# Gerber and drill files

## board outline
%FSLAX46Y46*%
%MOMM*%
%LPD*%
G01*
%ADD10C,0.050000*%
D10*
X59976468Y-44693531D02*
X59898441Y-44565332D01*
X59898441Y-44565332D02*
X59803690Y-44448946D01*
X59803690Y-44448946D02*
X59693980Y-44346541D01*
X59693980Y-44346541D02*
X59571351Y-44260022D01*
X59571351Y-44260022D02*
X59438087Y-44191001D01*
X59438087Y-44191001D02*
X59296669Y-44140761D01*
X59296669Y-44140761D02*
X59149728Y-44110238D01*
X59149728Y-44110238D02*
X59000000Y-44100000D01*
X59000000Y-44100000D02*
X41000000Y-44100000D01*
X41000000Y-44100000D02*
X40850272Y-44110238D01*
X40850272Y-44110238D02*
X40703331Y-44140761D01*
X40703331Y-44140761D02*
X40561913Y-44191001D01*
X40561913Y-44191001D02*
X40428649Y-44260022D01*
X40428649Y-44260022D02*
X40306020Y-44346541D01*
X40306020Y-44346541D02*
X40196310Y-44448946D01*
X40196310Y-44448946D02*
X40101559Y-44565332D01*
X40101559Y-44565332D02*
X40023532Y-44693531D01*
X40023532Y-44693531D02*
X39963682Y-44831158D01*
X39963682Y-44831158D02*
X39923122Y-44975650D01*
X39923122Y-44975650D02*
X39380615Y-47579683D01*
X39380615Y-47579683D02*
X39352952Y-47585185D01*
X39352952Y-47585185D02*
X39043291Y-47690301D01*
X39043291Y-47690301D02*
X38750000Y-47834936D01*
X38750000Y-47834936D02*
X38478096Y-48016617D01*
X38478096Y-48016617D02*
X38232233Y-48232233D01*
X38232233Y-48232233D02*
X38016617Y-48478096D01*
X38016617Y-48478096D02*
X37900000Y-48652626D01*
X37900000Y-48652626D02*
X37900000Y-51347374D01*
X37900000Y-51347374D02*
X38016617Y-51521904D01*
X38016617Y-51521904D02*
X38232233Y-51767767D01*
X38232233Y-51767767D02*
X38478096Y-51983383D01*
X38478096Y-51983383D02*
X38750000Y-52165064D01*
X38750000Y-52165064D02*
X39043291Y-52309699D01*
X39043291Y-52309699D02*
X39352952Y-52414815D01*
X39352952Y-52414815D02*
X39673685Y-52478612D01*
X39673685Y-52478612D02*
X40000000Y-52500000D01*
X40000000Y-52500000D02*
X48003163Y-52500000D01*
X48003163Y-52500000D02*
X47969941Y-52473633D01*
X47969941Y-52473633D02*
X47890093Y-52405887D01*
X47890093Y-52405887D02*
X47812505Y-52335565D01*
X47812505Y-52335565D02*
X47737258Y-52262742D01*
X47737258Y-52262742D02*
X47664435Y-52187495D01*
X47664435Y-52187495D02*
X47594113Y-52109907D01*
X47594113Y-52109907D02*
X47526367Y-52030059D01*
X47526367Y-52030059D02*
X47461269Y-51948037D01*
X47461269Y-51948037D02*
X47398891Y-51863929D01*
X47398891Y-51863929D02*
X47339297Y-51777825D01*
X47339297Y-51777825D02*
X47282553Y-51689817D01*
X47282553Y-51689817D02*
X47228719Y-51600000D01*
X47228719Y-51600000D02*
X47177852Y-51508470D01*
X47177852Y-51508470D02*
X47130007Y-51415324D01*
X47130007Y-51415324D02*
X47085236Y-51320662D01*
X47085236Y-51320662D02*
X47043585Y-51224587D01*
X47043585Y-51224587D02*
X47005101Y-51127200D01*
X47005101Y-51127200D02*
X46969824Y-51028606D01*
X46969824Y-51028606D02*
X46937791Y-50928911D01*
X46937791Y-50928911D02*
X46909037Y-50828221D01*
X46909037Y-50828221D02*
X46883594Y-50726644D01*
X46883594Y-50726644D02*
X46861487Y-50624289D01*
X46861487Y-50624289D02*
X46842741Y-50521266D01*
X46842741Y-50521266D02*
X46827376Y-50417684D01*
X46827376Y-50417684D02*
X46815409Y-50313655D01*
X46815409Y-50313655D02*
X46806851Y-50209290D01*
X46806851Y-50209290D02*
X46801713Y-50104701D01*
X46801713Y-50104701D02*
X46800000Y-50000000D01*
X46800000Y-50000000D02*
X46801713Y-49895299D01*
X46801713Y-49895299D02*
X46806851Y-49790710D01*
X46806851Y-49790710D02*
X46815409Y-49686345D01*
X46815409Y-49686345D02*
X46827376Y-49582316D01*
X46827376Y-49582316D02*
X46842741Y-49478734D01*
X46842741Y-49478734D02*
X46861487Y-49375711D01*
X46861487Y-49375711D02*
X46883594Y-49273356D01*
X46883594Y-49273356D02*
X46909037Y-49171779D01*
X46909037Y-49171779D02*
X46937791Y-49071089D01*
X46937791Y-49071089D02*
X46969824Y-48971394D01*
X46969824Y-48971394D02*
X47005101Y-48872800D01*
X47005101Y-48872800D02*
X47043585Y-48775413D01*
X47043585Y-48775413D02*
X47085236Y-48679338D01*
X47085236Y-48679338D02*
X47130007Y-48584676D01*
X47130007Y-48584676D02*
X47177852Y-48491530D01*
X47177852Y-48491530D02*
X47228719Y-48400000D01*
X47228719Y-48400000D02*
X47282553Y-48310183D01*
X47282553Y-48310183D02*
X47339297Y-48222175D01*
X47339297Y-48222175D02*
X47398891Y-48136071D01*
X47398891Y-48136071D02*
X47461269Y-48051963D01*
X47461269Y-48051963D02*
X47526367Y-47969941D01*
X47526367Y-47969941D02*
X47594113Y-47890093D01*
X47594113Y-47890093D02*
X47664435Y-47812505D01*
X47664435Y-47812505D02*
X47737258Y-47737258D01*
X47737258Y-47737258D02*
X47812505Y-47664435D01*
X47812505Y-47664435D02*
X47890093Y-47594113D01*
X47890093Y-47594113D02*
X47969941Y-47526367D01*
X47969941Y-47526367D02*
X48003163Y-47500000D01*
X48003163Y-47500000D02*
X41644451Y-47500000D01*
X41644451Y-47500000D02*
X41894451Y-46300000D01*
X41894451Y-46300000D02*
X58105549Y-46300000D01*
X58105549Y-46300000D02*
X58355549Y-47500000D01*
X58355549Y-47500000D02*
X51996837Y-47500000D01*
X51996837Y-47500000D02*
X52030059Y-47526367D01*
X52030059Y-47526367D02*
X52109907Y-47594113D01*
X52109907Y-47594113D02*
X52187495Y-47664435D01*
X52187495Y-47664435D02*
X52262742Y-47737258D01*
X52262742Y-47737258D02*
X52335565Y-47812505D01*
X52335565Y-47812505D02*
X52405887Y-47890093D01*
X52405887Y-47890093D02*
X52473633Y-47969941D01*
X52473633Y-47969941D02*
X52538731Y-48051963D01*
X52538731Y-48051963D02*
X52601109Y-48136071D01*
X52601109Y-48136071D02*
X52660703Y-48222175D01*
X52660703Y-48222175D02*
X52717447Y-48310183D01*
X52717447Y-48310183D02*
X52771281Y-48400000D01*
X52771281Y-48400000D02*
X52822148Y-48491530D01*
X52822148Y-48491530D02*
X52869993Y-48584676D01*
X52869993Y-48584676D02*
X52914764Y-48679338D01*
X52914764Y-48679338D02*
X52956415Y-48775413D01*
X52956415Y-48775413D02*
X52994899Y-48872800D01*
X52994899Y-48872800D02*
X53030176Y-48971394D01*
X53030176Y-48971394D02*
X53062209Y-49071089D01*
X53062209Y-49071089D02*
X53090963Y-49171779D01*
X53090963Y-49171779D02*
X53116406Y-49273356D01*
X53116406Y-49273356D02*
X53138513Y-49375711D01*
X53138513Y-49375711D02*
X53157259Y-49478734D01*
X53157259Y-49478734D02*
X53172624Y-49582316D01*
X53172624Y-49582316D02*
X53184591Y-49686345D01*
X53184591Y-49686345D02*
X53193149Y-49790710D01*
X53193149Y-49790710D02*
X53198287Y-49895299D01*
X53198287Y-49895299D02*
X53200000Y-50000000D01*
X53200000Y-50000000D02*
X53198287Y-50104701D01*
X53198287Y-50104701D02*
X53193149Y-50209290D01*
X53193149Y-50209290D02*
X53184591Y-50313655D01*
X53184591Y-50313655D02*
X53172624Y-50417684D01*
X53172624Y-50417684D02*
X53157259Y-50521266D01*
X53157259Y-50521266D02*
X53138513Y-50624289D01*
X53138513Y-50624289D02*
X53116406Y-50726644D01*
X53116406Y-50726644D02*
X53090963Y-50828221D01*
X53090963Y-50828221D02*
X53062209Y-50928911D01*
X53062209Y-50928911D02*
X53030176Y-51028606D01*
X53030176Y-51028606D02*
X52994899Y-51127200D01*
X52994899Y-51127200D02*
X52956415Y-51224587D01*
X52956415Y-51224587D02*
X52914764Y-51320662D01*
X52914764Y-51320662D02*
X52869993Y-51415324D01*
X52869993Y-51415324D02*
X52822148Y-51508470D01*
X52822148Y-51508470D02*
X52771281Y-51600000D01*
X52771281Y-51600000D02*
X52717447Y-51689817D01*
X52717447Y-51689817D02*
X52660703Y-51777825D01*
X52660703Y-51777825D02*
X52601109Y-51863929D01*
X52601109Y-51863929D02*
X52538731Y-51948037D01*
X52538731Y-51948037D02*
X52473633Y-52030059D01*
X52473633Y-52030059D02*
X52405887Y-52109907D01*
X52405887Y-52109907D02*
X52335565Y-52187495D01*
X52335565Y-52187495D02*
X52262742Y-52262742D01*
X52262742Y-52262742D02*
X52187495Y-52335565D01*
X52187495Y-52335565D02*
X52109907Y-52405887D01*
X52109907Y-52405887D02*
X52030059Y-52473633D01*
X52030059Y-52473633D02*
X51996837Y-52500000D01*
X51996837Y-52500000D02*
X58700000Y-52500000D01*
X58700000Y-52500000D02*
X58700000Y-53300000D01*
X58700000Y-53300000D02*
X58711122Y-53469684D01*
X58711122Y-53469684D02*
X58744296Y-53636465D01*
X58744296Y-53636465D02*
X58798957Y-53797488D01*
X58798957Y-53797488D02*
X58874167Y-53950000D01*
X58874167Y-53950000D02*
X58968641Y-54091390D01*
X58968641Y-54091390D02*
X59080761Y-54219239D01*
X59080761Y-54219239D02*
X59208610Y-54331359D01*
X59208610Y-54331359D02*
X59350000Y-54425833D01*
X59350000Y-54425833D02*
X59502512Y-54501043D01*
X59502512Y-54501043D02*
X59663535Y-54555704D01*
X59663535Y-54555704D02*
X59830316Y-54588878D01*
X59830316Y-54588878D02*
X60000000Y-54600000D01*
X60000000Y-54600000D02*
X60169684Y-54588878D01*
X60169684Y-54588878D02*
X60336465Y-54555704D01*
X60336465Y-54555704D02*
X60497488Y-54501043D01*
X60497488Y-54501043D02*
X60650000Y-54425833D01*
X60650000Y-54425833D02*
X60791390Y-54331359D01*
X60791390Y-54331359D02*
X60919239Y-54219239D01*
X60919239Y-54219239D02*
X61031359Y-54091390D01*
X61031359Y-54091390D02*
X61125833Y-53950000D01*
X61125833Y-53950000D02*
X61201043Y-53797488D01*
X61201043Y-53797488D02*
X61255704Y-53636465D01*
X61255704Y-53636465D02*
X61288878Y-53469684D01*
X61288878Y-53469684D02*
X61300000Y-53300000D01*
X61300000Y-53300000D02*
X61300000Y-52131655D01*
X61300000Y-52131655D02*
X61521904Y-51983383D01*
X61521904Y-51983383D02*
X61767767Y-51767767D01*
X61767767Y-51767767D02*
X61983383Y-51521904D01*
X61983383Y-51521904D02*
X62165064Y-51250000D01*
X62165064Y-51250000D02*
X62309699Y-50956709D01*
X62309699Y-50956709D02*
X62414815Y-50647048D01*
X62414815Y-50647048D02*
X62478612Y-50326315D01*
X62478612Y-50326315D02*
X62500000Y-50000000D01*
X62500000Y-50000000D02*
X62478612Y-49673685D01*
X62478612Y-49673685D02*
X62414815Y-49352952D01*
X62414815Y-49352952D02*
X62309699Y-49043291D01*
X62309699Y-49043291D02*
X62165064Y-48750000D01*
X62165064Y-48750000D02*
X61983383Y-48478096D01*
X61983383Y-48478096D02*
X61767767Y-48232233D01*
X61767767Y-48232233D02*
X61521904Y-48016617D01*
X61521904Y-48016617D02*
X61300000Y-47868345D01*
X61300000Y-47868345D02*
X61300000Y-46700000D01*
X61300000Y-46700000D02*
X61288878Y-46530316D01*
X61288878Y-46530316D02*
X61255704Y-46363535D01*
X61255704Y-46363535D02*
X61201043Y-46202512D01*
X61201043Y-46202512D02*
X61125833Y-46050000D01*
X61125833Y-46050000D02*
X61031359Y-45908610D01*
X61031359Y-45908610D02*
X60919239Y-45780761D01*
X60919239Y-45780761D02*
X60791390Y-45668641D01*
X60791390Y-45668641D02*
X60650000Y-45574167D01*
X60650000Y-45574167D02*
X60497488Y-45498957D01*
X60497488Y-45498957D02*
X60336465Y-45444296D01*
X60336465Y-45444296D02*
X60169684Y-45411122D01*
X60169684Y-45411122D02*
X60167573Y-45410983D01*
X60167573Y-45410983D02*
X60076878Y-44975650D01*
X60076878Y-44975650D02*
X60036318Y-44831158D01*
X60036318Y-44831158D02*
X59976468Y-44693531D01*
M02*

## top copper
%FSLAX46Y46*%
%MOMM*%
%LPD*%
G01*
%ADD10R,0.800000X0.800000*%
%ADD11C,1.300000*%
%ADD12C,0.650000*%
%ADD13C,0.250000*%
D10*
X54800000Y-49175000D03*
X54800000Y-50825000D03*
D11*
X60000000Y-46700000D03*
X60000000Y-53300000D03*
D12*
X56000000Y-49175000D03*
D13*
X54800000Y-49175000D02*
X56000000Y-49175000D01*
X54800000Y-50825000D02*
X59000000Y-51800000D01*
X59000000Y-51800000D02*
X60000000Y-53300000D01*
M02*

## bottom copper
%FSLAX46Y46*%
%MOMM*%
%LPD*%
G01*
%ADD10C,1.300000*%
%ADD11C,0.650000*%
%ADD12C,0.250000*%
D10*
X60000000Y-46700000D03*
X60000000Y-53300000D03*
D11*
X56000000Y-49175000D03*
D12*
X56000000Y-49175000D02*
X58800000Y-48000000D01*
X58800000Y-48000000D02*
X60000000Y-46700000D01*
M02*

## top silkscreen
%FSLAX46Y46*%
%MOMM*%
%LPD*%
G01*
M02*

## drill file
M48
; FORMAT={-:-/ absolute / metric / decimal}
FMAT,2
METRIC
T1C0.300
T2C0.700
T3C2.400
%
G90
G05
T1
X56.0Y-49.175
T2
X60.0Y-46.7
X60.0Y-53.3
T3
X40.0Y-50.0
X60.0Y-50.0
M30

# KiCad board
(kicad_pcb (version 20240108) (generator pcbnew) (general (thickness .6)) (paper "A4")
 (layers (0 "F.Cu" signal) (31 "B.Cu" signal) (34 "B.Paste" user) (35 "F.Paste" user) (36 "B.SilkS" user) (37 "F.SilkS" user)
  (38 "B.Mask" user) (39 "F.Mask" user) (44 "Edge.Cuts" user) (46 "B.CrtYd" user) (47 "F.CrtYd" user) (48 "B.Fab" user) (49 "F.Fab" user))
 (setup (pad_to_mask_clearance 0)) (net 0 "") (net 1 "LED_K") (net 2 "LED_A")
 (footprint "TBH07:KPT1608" (layer "F.Cu") (at 54.8 50)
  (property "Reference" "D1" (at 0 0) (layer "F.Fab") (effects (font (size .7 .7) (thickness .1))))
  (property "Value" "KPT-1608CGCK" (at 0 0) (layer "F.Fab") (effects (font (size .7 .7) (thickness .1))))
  (pad "1" smd rect (at 0 -.825) (size .8 .8) (layers "F.Cu" "F.Paste" "F.Mask") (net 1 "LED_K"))
  (pad "2" smd rect (at 0 .825) (size .8 .8) (layers "F.Cu" "F.Paste" "F.Mask") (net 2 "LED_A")))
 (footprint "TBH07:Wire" (layer "F.Cu") (at 60 46.7)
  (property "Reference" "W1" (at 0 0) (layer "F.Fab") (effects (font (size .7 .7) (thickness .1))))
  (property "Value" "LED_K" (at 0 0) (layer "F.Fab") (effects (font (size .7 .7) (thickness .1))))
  (pad "1" thru_hole circle (at 0 0) (size 1.3 1.3) (drill .7) (layers "*.Cu" "*.Mask") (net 1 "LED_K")))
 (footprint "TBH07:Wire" (layer "F.Cu") (at 60 53.3)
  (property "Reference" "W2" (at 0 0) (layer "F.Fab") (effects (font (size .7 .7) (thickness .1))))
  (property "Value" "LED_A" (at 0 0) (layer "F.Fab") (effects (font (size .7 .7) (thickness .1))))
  (pad "1" thru_hole circle (at 0 0) (size 1.3 1.3) (drill .7) (layers "*.Cu" "*.Mask") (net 2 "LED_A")))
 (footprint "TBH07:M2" (layer "F.Cu") (at 40 50)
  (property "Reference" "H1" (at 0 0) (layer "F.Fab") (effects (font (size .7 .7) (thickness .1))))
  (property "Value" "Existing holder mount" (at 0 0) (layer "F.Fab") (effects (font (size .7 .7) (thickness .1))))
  (pad "" np_thru_hole circle (at 0 0) (size 2.4 2.4) (drill 2.4) (layers "*.Cu" "*.Mask")))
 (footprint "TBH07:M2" (layer "F.Cu") (at 60 50)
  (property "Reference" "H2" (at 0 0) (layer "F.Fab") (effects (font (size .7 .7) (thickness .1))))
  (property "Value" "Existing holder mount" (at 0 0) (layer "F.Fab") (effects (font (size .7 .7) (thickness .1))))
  (pad "" np_thru_hole circle (at 0 0) (size 2.4 2.4) (drill 2.4) (layers "*.Cu" "*.Mask")))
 (segment (start 54.8 49.175) (end 56 49.175) (width .25) (layer "F.Cu") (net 1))
 (via (at 56 49.175) (size .65) (drill .3) (layers "F.Cu" "B.Cu") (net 1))
 (segment (start 56 49.175) (end 58.8 48.0) (width .25) (layer "B.Cu") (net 1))
 (segment (start 58.8 48.0) (end 60 46.7) (width .25) (layer "B.Cu") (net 1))
 (segment (start 54.8 50.825) (end 59.0 51.8) (width .25) (layer "F.Cu") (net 2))
 (segment (start 59.0 51.8) (end 60 53.3) (width .25) (layer "F.Cu") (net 2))
 (gr_line (start 59.97646762268844 44.69353086782984) (end 59.89844084614742 44.56533154641664) (stroke (width .05) (type default))
  (layer "Edge.Cuts"))
 (gr_line (start 59.89844084614742 44.56533154641664) (end 59.80369026607012 44.448946102983186) (stroke (width .05) (type default))
  (layer "Edge.Cuts"))
 (gr_line (start 59.80369026607012 44.448946102983186) (end 59.69397959354886 44.34654096540152) (stroke (width .05) (type default))
  (layer "Edge.Cuts"))
 (gr_line (start 59.69397959354886 44.34654096540152) (end 59.57135101059367 44.26002232861967) (stroke (width .05) (type default))
  (layer "Edge.Cuts"))
 (gr_line (start 59.57135101059367 44.26002232861967) (end 59.4380871564435 44.19100067227017) (stroke (width .05) (type default))
  (layer "Edge.Cuts"))
 (gr_line (start 59.4380871564435 44.19100067227017) (end 59.29666863794614 44.14076078279778) (stroke (width .05) (type default))
  (layer "Edge.Cuts"))
 (gr_line (start 59.29666863794614 44.14076078279778) (end 59.14972785491944 44.110237838121904) (stroke (width .05) (type default))
  (layer "Edge.Cuts"))
 (gr_line (start 59.14972785491944 44.110237838121904) (end 59.0 44.1) (stroke (width .05) (type default)) (layer "Edge.Cuts"))
 (gr_line (start 59.0 44.1) (end 41.0 44.1) (stroke (width .05) (type default)) (layer "Edge.Cuts"))
 (gr_line (start 41.0 44.1) (end 40.85027214508056 44.110237838121904) (stroke (width .05) (type default)) (layer "Edge.Cuts"))
 (gr_line (start 40.85027214508056 44.110237838121904) (end 40.70333136205386 44.14076078279778) (stroke (width .05) (type default))
  (layer "Edge.Cuts"))
 (gr_line (start 40.70333136205386 44.14076078279778) (end 40.5619128435565 44.19100067227017) (stroke (width .05) (type default))
  (layer "Edge.Cuts"))
 (gr_line (start 40.5619128435565 44.19100067227017) (end 40.42864898940633 44.26002232861967) (stroke (width .05) (type default))
  (layer "Edge.Cuts"))
 (gr_line (start 40.42864898940633 44.26002232861967) (end 40.30602040645114 44.34654096540152) (stroke (width .05) (type default))
  (layer "Edge.Cuts"))
 (gr_line (start 40.30602040645114 44.34654096540152) (end 40.19630973392988 44.448946102983186) (stroke (width .05) (type default))
  (layer "Edge.Cuts"))
 (gr_line (start 40.19630973392988 44.448946102983186) (end 40.10155915385258 44.56533154641664) (stroke (width .05) (type default))
  (layer "Edge.Cuts"))
 (gr_line (start 40.10155915385258 44.56533154641664) (end 40.02353237731156 44.69353086782984) (stroke (width .05) (type default))
  (layer "Edge.Cuts"))
 (gr_line (start 40.02353237731156 44.69353086782984) (end 39.9636818143203 44.831157732859225) (stroke (width .05) (type default))
  (layer "Edge.Cuts"))
 (gr_line (start 39.9636818143203 44.831157732859225) (end 39.92312153828863 44.9756503204768) (stroke (width .05) (type default))
  (layer "Edge.Cuts"))
 (gr_line (start 39.92312153828863 44.9756503204768) (end 39.3806147187135 47.57968305443743) (stroke (width .05) (type default))
  (layer "Edge.Cuts"))
 (gr_line (start 39.3806147187135 47.57968305443743) (end 39.3529523872437 47.58518543427733) (stroke (width .05) (type default))
  (layer "Edge.Cuts"))
 (gr_line (start 39.3529523872437 47.58518543427733) (end 39.043291419087275 47.69030116872178) (stroke (width .05) (type default))
  (layer "Edge.Cuts"))
 (gr_line (start 39.043291419087275 47.69030116872178) (end 38.75 47.8349364905389) (stroke (width .05) (type default)) (layer "Edge.Cuts"))
 (gr_line (start 38.75 47.8349364905389) (end 38.4780964274782 48.01661664927191) (stroke (width .05) (type default)) (layer "Edge.Cuts"))
 (gr_line (start 38.4780964274782 48.01661664927191) (end 38.23223304703363 48.23223304703363) (stroke (width .05) (type default))
  (layer "Edge.Cuts"))
 (gr_line (start 38.23223304703363 48.23223304703363) (end 38.01661664927191 48.4780964274782) (stroke (width .05) (type default))
  (layer "Edge.Cuts"))
 (gr_line (start 38.01661664927191 48.4780964274782) (end 37.9 48.652625576801285) (stroke (width .05) (type default)) (layer "Edge.Cuts"))
 (gr_line (start 37.9 48.652625576801285) (end 37.9 51.347374423198715) (stroke (width .05) (type default)) (layer "Edge.Cuts"))
 (gr_line (start 37.9 51.347374423198715) (end 38.01661664927191 51.5219035725218) (stroke (width .05) (type default)) (layer "Edge.Cuts"))
 (gr_line (start 38.01661664927191 51.5219035725218) (end 38.23223304703363 51.76776695296637) (stroke (width .05) (type default))
  (layer "Edge.Cuts"))
 (gr_line (start 38.23223304703363 51.76776695296637) (end 38.4780964274782 51.98338335072809) (stroke (width .05) (type default))
  (layer "Edge.Cuts"))
 (gr_line (start 38.4780964274782 51.98338335072809) (end 38.75 52.1650635094611) (stroke (width .05) (type default)) (layer "Edge.Cuts"))
 (gr_line (start 38.75 52.1650635094611) (end 39.043291419087275 52.30969883127822) (stroke (width .05) (type default)) (layer "Edge.Cuts"))
 (gr_line (start 39.043291419087275 52.30969883127822) (end 39.3529523872437 52.41481456572267) (stroke (width .05) (type default))
  (layer "Edge.Cuts"))
 (gr_line (start 39.3529523872437 52.41481456572267) (end 39.67368451944987 52.478612153434526) (stroke (width .05) (type default))
  (layer "Edge.Cuts"))
 (gr_line (start 39.67368451944987 52.478612153434526) (end 40.0 52.5) (stroke (width .05) (type default)) (layer "Edge.Cuts"))
 (gr_line (start 40.0 52.5) (end 48.00316310634037 52.5) (stroke (width .05) (type default)) (layer "Edge.Cuts"))
 (gr_line (start 48.00316310634037 52.5) (end 47.969941490676334 52.47363345076076) (stroke (width .05) (type default)) (layer "Edge.Cuts"))
 (gr_line (start 47.969941490676334 52.47363345076076) (end 47.89009339167978 52.40588738393273) (stroke (width .05) (type default))
  (layer "Edge.Cuts"))
 (gr_line (start 47.89009339167978 52.40588738393273) (end 47.812504633526814 52.33556503263307) (stroke (width .05) (type default))
  (layer "Edge.Cuts"))
 (gr_line (start 47.812504633526814 52.33556503263307) (end 47.737258300203045 52.26274169979695) (stroke (width .05) (type default))
  (layer "Edge.Cuts"))
 (gr_line (start 47.737258300203045 52.26274169979695) (end 47.66443496736692 52.187495366473186) (stroke (width .05) (type default))
  (layer "Edge.Cuts"))
 (gr_line (start 47.66443496736692 52.187495366473186) (end 47.59411261606727 52.109906608320216) (stroke (width .05) (type default))
  (layer "Edge.Cuts"))
 (gr_line (start 47.59411261606727 52.109906608320216) (end 47.52636654923924 52.030058509323666) (stroke (width .05) (type default))
  (layer "Edge.Cuts"))
 (gr_line (start 47.52636654923924 52.030058509323666) (end 47.461269311068044 51.9480365728279) (stroke (width .05) (type default))
  (layer "Edge.Cuts"))
 (gr_line (start 47.461269311068044 51.9480365728279) (end 47.39889060930683 51.86392862997697) (stroke (width .05) (type default))
  (layer "Edge.Cuts"))
 (gr_line (start 47.39889060930683 51.86392862997697) (end 47.33929724063185 51.77782474566273) (stroke (width .05) (type default))
  (layer "Edge.Cuts"))
 (gr_line (start 47.33929724063185 51.77782474566273) (end 47.28255301911494 51.68981712208117) (stroke (width .05) (type default))
  (layer "Edge.Cuts"))
 (gr_line (start 47.28255301911494 51.68981712208117) (end 47.2287187078898 51.6) (stroke (width .05) (type default)) (layer "Edge.Cuts"))
 (gr_line (start 47.2287187078898 51.6) (end 47.17785195408526 51.50846955784319) (stroke (width .05) (type default)) (layer "Edge.Cuts"))
 (gr_line (start 47.17785195408526 51.50846955784319) (end 47.1300072270954 51.415323808700805) (stroke (width .05) (type default))
  (layer "Edge.Cuts"))
 (gr_line (start 47.1300072270954 51.415323808700805) (end 47.08523576025224 51.320662495374066) (stroke (width .05) (type default))
  (layer "Edge.Cuts"))
 (gr_line (start 47.08523576025224 51.320662495374066) (end 47.04358549596388 51.22458698356829) (stroke (width .05) (type default))
  (layer "Edge.Cuts"))
 (gr_line (start 47.04358549596388 51.22458698356829) (end 47.00510103437656 51.12720015334795) (stroke (width .05) (type default))
  (layer "Edge.Cuts"))
 (gr_line (start 47.00510103437656 51.12720015334795) (end 46.969823585615664 51.02860628897012) (stroke (width .05) (type default))
  (layer "Edge.Cuts"))
 (gr_line (start 46.969823585615664 51.02860628897012) (end 46.937790925656934 50.92891096721428) (stroke (width .05) (type default))
  (layer "Edge.Cuts"))
 (gr_line (start 46.937790925656934 50.92891096721428) (end 46.90903735587498 50.828220944328066) (stroke (width .05) (type default))
  (layer "Edge.Cuts"))
 (gr_line (start 46.90903735587498 50.828220944328066) (end 46.883593666312535 50.726644041709996) (stroke (width .05) (type default))
  (layer "Edge.Cuts"))
 (gr_line (start 46.883593666312535 50.726644041709996) (end 46.86148710270966 50.62428903045161) (stroke (width .05) (type default))
  (layer "Edge.Cuts"))
 (gr_line (start 46.86148710270966 50.62428903045161) (end 46.842741337328384 50.521265514862684) (stroke (width .05) (type default))
  (layer "Edge.Cuts"))
 (gr_line (start 46.842741337328384 50.521265514862684) (end 46.827376443603804 50.41768381510416) (stroke (width .05) (type default))
  (layer "Edge.Cuts"))
 (gr_line (start 46.827376443603804 50.41768381510416) (end 46.815408874648966 50.31365484905459) (stroke (width .05) (type default))
  (layer "Edge.Cuts"))
 (gr_line (start 46.815408874648966 50.31365484905459) (end 46.80685144563647 50.20929001353646) (stroke (width .05) (type default))
  (layer "Edge.Cuts"))
 (gr_line (start 46.80685144563647 50.20929001353646) (end 46.80171332007563 50.10470106502968) (stroke (width .05) (type default))
  (layer "Edge.Cuts"))
 (gr_line (start 46.80171332007563 50.10470106502968) (end 46.8 50.0) (stroke (width .05) (type default)) (layer "Edge.Cuts"))
 (gr_line (start 46.8 50.0) (end 46.80171332007563 49.89529893497031) (stroke (width .05) (type default)) (layer "Edge.Cuts"))
 (gr_line (start 46.80171332007563 49.89529893497031) (end 46.80685144563647 49.79070998646354) (stroke (width .05) (type default))
  (layer "Edge.Cuts"))
 (gr_line (start 46.80685144563647 49.79070998646354) (end 46.815408874648966 49.68634515094541) (stroke (width .05) (type default))
  (layer "Edge.Cuts"))
 (gr_line (start 46.815408874648966 49.68634515094541) (end 46.827376443603804 49.58231618489583) (stroke (width .05) (type default))
  (layer "Edge.Cuts"))
 (gr_line (start 46.827376443603804 49.58231618489583) (end 46.842741337328384 49.478734485137316) (stroke (width .05) (type default))
  (layer "Edge.Cuts"))
 (gr_line (start 46.842741337328384 49.478734485137316) (end 46.86148710270966 49.375710969548386) (stroke (width .05) (type default))
  (layer "Edge.Cuts"))
 (gr_line (start 46.86148710270966 49.375710969548386) (end 46.883593666312535 49.273355958290004) (stroke (width .05) (type default))
  (layer "Edge.Cuts"))
 (gr_line (start 46.883593666312535 49.273355958290004) (end 46.90903735587498 49.171779055671934) (stroke (width .05) (type default))
  (layer "Edge.Cuts"))
 (gr_line (start 46.90903735587498 49.171779055671934) (end 46.937790925656934 49.07108903278572) (stroke (width .05) (type default))
  (layer "Edge.Cuts"))
 (gr_line (start 46.937790925656934 49.07108903278572) (end 46.969823585615664 48.97139371102988) (stroke (width .05) (type default))
  (layer "Edge.Cuts"))
 (gr_line (start 46.969823585615664 48.97139371102988) (end 47.00510103437656 48.87279984665205) (stroke (width .05) (type default))
  (layer "Edge.Cuts"))
 (gr_line (start 47.00510103437656 48.87279984665205) (end 47.04358549596388 48.77541301643171) (stroke (width .05) (type default))
  (layer "Edge.Cuts"))
 (gr_line (start 47.04358549596388 48.77541301643171) (end 47.08523576025224 48.679337504625934) (stroke (width .05) (type default))
  (layer "Edge.Cuts"))
 (gr_line (start 47.08523576025224 48.679337504625934) (end 47.1300072270954 48.584676191299195) (stroke (width .05) (type default))
  (layer "Edge.Cuts"))
 (gr_line (start 47.1300072270954 48.584676191299195) (end 47.17785195408526 48.49153044215681) (stroke (width .05) (type default))
  (layer "Edge.Cuts"))
 (gr_line (start 47.17785195408526 48.49153044215681) (end 47.2287187078898 48.4) (stroke (width .05) (type default)) (layer "Edge.Cuts"))
 (gr_line (start 47.2287187078898 48.4) (end 47.28255301911495 48.31018287791882) (stroke (width .05) (type default)) (layer "Edge.Cuts"))
 (gr_line (start 47.28255301911495 48.31018287791882) (end 47.33929724063186 48.22217525433727) (stroke (width .05) (type default))
  (layer "Edge.Cuts"))
 (gr_line (start 47.33929724063186 48.22217525433727) (end 47.39889060930683 48.13607137002303) (stroke (width .05) (type default))
  (layer "Edge.Cuts"))
 (gr_line (start 47.39889060930683 48.13607137002303) (end 47.46126931106805 48.05196342717209) (stroke (width .05) (type default))
  (layer "Edge.Cuts"))
 (gr_line (start 47.46126931106805 48.05196342717209) (end 47.52636654923924 47.969941490676334) (stroke (width .05) (type default))
  (layer "Edge.Cuts"))
 (gr_line (start 47.52636654923924 47.969941490676334) (end 47.59411261606727 47.89009339167978) (stroke (width .05) (type default))
  (layer "Edge.Cuts"))
 (gr_line (start 47.59411261606727 47.89009339167978) (end 47.66443496736693 47.812504633526814) (stroke (width .05) (type default))
  (layer "Edge.Cuts"))
 (gr_line (start 47.66443496736693 47.812504633526814) (end 47.737258300203045 47.737258300203045) (stroke (width .05) (type default))
  (layer "Edge.Cuts"))
 (gr_line (start 47.737258300203045 47.737258300203045) (end 47.812504633526814 47.66443496736692) (stroke (width .05) (type default))
  (layer "Edge.Cuts"))
 (gr_line (start 47.812504633526814 47.66443496736692) (end 47.890093391679784 47.59411261606727) (stroke (width .05) (type default))
  (layer "Edge.Cuts"))
 (gr_line (start 47.890093391679784 47.59411261606727) (end 47.969941490676334 47.52636654923924) (stroke (width .05) (type default))
  (layer "Edge.Cuts"))
 (gr_line (start 47.969941490676334 47.52636654923924) (end 48.00316310634037 47.5) (stroke (width .05) (type default)) (layer "Edge.Cuts"))
 (gr_line (start 48.00316310634037 47.5) (end 41.64445131161203 47.5) (stroke (width .05) (type default)) (layer "Edge.Cuts"))
 (gr_line (start 41.64445131161203 47.5) (end 41.89445131161203 46.3) (stroke (width .05) (type default)) (layer "Edge.Cuts"))
 (gr_line (start 41.89445131161203 46.3) (end 58.10554868838797 46.3) (stroke (width .05) (type default)) (layer "Edge.Cuts"))
 (gr_line (start 58.10554868838797 46.3) (end 58.35554868838797 47.5) (stroke (width .05) (type default)) (layer "Edge.Cuts"))
 (gr_line (start 58.35554868838797 47.5) (end 51.99683689365963 47.5) (stroke (width .05) (type default)) (layer "Edge.Cuts"))
 (gr_line (start 51.99683689365963 47.5) (end 52.030058509323666 47.52636654923924) (stroke (width .05) (type default)) (layer "Edge.Cuts"))
 (gr_line (start 52.030058509323666 47.52636654923924) (end 52.10990660832022 47.59411261606727) (stroke (width .05) (type default))
  (layer "Edge.Cuts"))
 (gr_line (start 52.10990660832022 47.59411261606727) (end 52.187495366473186 47.66443496736693) (stroke (width .05) (type default))
  (layer "Edge.Cuts"))
 (gr_line (start 52.187495366473186 47.66443496736693) (end 52.262741699796955 47.737258300203045) (stroke (width .05) (type default))
  (layer "Edge.Cuts"))
 (gr_line (start 52.262741699796955 47.737258300203045) (end 52.33556503263308 47.812504633526814) (stroke (width .05) (type default))
  (layer "Edge.Cuts"))
 (gr_line (start 52.33556503263308 47.812504633526814) (end 52.40588738393273 47.89009339167978) (stroke (width .05) (type default))
  (layer "Edge.Cuts"))
 (gr_line (start 52.40588738393273 47.89009339167978) (end 52.47363345076076 47.969941490676334) (stroke (width .05) (type default))
  (layer "Edge.Cuts"))
 (gr_line (start 52.47363345076076 47.969941490676334) (end 52.538730688931956 48.0519634271721) (stroke (width .05) (type default))
  (layer "Edge.Cuts"))
 (gr_line (start 52.538730688931956 48.0519634271721) (end 52.60110939069317 48.13607137002303) (stroke (width .05) (type default))
  (layer "Edge.Cuts"))
 (gr_line (start 52.60110939069317 48.13607137002303) (end 52.66070275936814 48.22217525433727) (stroke (width .05) (type default))
  (layer "Edge.Cuts"))
 (gr_line (start 52.66070275936814 48.22217525433727) (end 52.71744698088505 48.31018287791882) (stroke (width .05) (type default))
  (layer "Edge.Cuts"))
 (gr_line (start 52.71744698088505 48.31018287791882) (end 52.7712812921102 48.4) (stroke (width .05) (type default)) (layer "Edge.Cuts"))
 (gr_line (start 52.7712812921102 48.4) (end 52.82214804591474 48.49153044215681) (stroke (width .05) (type default)) (layer "Edge.Cuts"))
 (gr_line (start 52.82214804591474 48.49153044215681) (end 52.8699927729046 48.584676191299195) (stroke (width .05) (type default))
  (layer "Edge.Cuts"))
 (gr_line (start 52.8699927729046 48.584676191299195) (end 52.91476423974776 48.679337504625934) (stroke (width .05) (type default))
  (layer "Edge.Cuts"))
 (gr_line (start 52.91476423974776 48.679337504625934) (end 52.95641450403612 48.77541301643171) (stroke (width .05) (type default))
  (layer "Edge.Cuts"))
 (gr_line (start 52.95641450403612 48.77541301643171) (end 52.99489896562344 48.87279984665205) (stroke (width .05) (type default))
  (layer "Edge.Cuts"))
 (gr_line (start 52.99489896562344 48.87279984665205) (end 53.030176414384336 48.97139371102988) (stroke (width .05) (type default))
  (layer "Edge.Cuts"))
 (gr_line (start 53.030176414384336 48.97139371102988) (end 53.062209074343066 49.07108903278572) (stroke (width .05) (type default))
  (layer "Edge.Cuts"))
 (gr_line (start 53.062209074343066 49.07108903278572) (end 53.09096264412502 49.171779055671934) (stroke (width .05) (type default))
  (layer "Edge.Cuts"))
 (gr_line (start 53.09096264412502 49.171779055671934) (end 53.116406333687465 49.273355958290004) (stroke (width .05) (type default))
  (layer "Edge.Cuts"))
 (gr_line (start 53.116406333687465 49.273355958290004) (end 53.13851289729034 49.375710969548386) (stroke (width .05) (type default))
  (layer "Edge.Cuts"))
 (gr_line (start 53.13851289729034 49.375710969548386) (end 53.157258662671616 49.478734485137316) (stroke (width .05) (type default))
  (layer "Edge.Cuts"))
 (gr_line (start 53.157258662671616 49.478734485137316) (end 53.172623556396196 49.58231618489584) (stroke (width .05) (type default))
  (layer "Edge.Cuts"))
 (gr_line (start 53.172623556396196 49.58231618489584) (end 53.184591125351034 49.68634515094541) (stroke (width .05) (type default))
  (layer "Edge.Cuts"))
 (gr_line (start 53.184591125351034 49.68634515094541) (end 53.19314855436353 49.79070998646354) (stroke (width .05) (type default))
  (layer "Edge.Cuts"))
 (gr_line (start 53.19314855436353 49.79070998646354) (end 53.19828667992437 49.89529893497031) (stroke (width .05) (type default))
  (layer "Edge.Cuts"))
 (gr_line (start 53.19828667992437 49.89529893497031) (end 53.2 50.0) (stroke (width .05) (type default)) (layer "Edge.Cuts"))
 (gr_line (start 53.2 50.0) (end 53.19828667992437 50.10470106502969) (stroke (width .05) (type default)) (layer "Edge.Cuts"))
 (gr_line (start 53.19828667992437 50.10470106502969) (end 53.19314855436353 50.20929001353646) (stroke (width .05) (type default))
  (layer "Edge.Cuts"))
 (gr_line (start 53.19314855436353 50.20929001353646) (end 53.184591125351034 50.31365484905459) (stroke (width .05) (type default))
  (layer "Edge.Cuts"))
 (gr_line (start 53.184591125351034 50.31365484905459) (end 53.17262355639619 50.41768381510417) (stroke (width .05) (type default))
  (layer "Edge.Cuts"))
 (gr_line (start 53.17262355639619 50.41768381510417) (end 53.157258662671616 50.521265514862684) (stroke (width .05) (type default))
  (layer "Edge.Cuts"))
 (gr_line (start 53.157258662671616 50.521265514862684) (end 53.13851289729034 50.624289030451614) (stroke (width .05) (type default))
  (layer "Edge.Cuts"))
 (gr_line (start 53.13851289729034 50.624289030451614) (end 53.116406333687465 50.726644041709996) (stroke (width .05) (type default))
  (layer "Edge.Cuts"))
 (gr_line (start 53.116406333687465 50.726644041709996) (end 53.09096264412502 50.828220944328066) (stroke (width .05) (type default))
  (layer "Edge.Cuts"))
 (gr_line (start 53.09096264412502 50.828220944328066) (end 53.062209074343066 50.928910967214286) (stroke (width .05) (type default))
  (layer "Edge.Cuts"))
 (gr_line (start 53.062209074343066 50.928910967214286) (end 53.030176414384336 51.02860628897012) (stroke (width .05) (type default))
  (layer "Edge.Cuts"))
 (gr_line (start 53.030176414384336 51.02860628897012) (end 52.99489896562344 51.12720015334795) (stroke (width .05) (type default))
  (layer "Edge.Cuts"))
 (gr_line (start 52.99489896562344 51.12720015334795) (end 52.95641450403612 51.22458698356829) (stroke (width .05) (type default))
  (layer "Edge.Cuts"))
 (gr_line (start 52.95641450403612 51.22458698356829) (end 52.91476423974776 51.320662495374066) (stroke (width .05) (type default))
  (layer "Edge.Cuts"))
 (gr_line (start 52.91476423974776 51.320662495374066) (end 52.8699927729046 51.415323808700805) (stroke (width .05) (type default))
  (layer "Edge.Cuts"))
 (gr_line (start 52.8699927729046 51.415323808700805) (end 52.82214804591474 51.50846955784319) (stroke (width .05) (type default))
  (layer "Edge.Cuts"))
 (gr_line (start 52.82214804591474 51.50846955784319) (end 52.7712812921102 51.6) (stroke (width .05) (type default)) (layer "Edge.Cuts"))
 (gr_line (start 52.7712812921102 51.6) (end 52.71744698088505 51.68981712208118) (stroke (width .05) (type default)) (layer "Edge.Cuts"))
 (gr_line (start 52.71744698088505 51.68981712208118) (end 52.66070275936814 51.77782474566273) (stroke (width .05) (type default))
  (layer "Edge.Cuts"))
 (gr_line (start 52.66070275936814 51.77782474566273) (end 52.60110939069317 51.86392862997697) (stroke (width .05) (type default))
  (layer "Edge.Cuts"))
 (gr_line (start 52.60110939069317 51.86392862997697) (end 52.53873068893195 51.94803657282791) (stroke (width .05) (type default))
  (layer "Edge.Cuts"))
 (gr_line (start 52.53873068893195 51.94803657282791) (end 52.47363345076076 52.030058509323666) (stroke (width .05) (type default))
  (layer "Edge.Cuts"))
 (gr_line (start 52.47363345076076 52.030058509323666) (end 52.40588738393273 52.10990660832022) (stroke (width .05) (type default))
  (layer "Edge.Cuts"))
 (gr_line (start 52.40588738393273 52.10990660832022) (end 52.33556503263307 52.18749536647319) (stroke (width .05) (type default))
  (layer "Edge.Cuts"))
 (gr_line (start 52.33556503263307 52.18749536647319) (end 52.262741699796955 52.262741699796955) (stroke (width .05) (type default))
  (layer "Edge.Cuts"))
 (gr_line (start 52.262741699796955 52.262741699796955) (end 52.187495366473186 52.33556503263308) (stroke (width .05) (type default))
  (layer "Edge.Cuts"))
 (gr_line (start 52.187495366473186 52.33556503263308) (end 52.109906608320216 52.40588738393273) (stroke (width .05) (type default))
  (layer "Edge.Cuts"))
 (gr_line (start 52.109906608320216 52.40588738393273) (end 52.030058509323666 52.47363345076076) (stroke (width .05) (type default))
  (layer "Edge.Cuts"))
 (gr_line (start 52.030058509323666 52.47363345076076) (end 51.99683689365963 52.5) (stroke (width .05) (type default)) (layer "Edge.Cuts"))
 (gr_line (start 51.99683689365963 52.5) (end 58.7 52.5) (stroke (width .05) (type default)) (layer "Edge.Cuts"))
 (gr_line (start 58.7 52.5) (end 58.7 53.3) (stroke (width .05) (type default)) (layer "Edge.Cuts"))
 (gr_line (start 58.7 53.3) (end 58.71112168021405 53.46968404988607) (stroke (width .05) (type default)) (layer "Edge.Cuts"))
 (gr_line (start 58.71112168021405 53.46968404988607) (end 58.74429642582421 53.63646475863328) (stroke (width .05) (type default))
  (layer "Edge.Cuts"))
 (gr_line (start 58.74429642582421 53.63646475863328) (end 58.79895660773533 53.79748846207462) (stroke (width .05) (type default))
  (layer "Edge.Cuts"))
 (gr_line (start 58.79895660773533 53.79748846207462) (end 58.87416697508023 53.95) (stroke (width .05) (type default)) (layer "Edge.Cuts"))
 (gr_line (start 58.87416697508023 53.95) (end 58.96864065762139 54.091389857711334) (stroke (width .05) (type default)) (layer "Edge.Cuts"))
 (gr_line (start 58.96864065762139 54.091389857711334) (end 59.08076118445749 54.21923881554251) (stroke (width .05) (type default))
  (layer "Edge.Cuts"))
 (gr_line (start 59.08076118445749 54.21923881554251) (end 59.20861014228866 54.331359342378605) (stroke (width .05) (type default))
  (layer "Edge.Cuts"))
 (gr_line (start 59.20861014228866 54.331359342378605) (end 59.35 54.42583302491977) (stroke (width .05) (type default)) (layer "Edge.Cuts"))
 (gr_line (start 59.35 54.42583302491977) (end 59.502511537925386 54.50104339226467) (stroke (width .05) (type default)) (layer "Edge.Cuts"))
 (gr_line (start 59.502511537925386 54.50104339226467) (end 59.66353524136672 54.55570357417579) (stroke (width .05) (type default))
  (layer "Edge.Cuts"))
 (gr_line (start 59.66353524136672 54.55570357417579) (end 59.830315950113935 54.588878319785955) (stroke (width .05) (type default))
  (layer "Edge.Cuts"))
 (gr_line (start 59.830315950113935 54.588878319785955) (end 60.0 54.6) (stroke (width .05) (type default)) (layer "Edge.Cuts"))
 (gr_line (start 60.0 54.6) (end 60.169684049886065 54.588878319785955) (stroke (width .05) (type default)) (layer "Edge.Cuts"))
 (gr_line (start 60.169684049886065 54.588878319785955) (end 60.33646475863328 54.55570357417579) (stroke (width .05) (type default))
  (layer "Edge.Cuts"))
 (gr_line (start 60.33646475863328 54.55570357417579) (end 60.497488462074614 54.50104339226468) (stroke (width .05) (type default))
  (layer "Edge.Cuts"))
 (gr_line (start 60.497488462074614 54.50104339226468) (end 60.65 54.42583302491977) (stroke (width .05) (type default)) (layer "Edge.Cuts"))
 (gr_line (start 60.65 54.42583302491977) (end 60.79138985771134 54.331359342378605) (stroke (width .05) (type default)) (layer "Edge.Cuts"))
 (gr_line (start 60.79138985771134 54.331359342378605) (end 60.91923881554251 54.21923881554251) (stroke (width .05) (type default))
  (layer "Edge.Cuts"))
 (gr_line (start 60.91923881554251 54.21923881554251) (end 61.03135934237861 54.091389857711334) (stroke (width .05) (type default))
  (layer "Edge.Cuts"))
 (gr_line (start 61.03135934237861 54.091389857711334) (end 61.12583302491977 53.95) (stroke (width .05) (type default)) (layer "Edge.Cuts"))
 (gr_line (start 61.12583302491977 53.95) (end 61.20104339226467 53.79748846207462) (stroke (width .05) (type default)) (layer "Edge.Cuts"))
 (gr_line (start 61.20104339226467 53.79748846207462) (end 61.25570357417579 53.63646475863328) (stroke (width .05) (type default))
  (layer "Edge.Cuts"))
 (gr_line (start 61.25570357417579 53.63646475863328) (end 61.28887831978595 53.46968404988607) (stroke (width .05) (type default))
  (layer "Edge.Cuts"))
 (gr_line (start 61.28887831978595 53.46968404988607) (end 61.3 53.3) (stroke (width .05) (type default)) (layer "Edge.Cuts"))
 (gr_line (start 61.3 53.3) (end 61.3 52.13165457756513) (stroke (width .05) (type default)) (layer "Edge.Cuts"))
 (gr_line (start 61.3 52.13165457756513) (end 61.5219035725218 51.98338335072809) (stroke (width .05) (type default)) (layer "Edge.Cuts"))
 (gr_line (start 61.5219035725218 51.98338335072809) (end 61.76776695296637 51.76776695296637) (stroke (width .05) (type default))
  (layer "Edge.Cuts"))
 (gr_line (start 61.76776695296637 51.76776695296637) (end 61.98338335072809 51.5219035725218) (stroke (width .05) (type default))
  (layer "Edge.Cuts"))
 (gr_line (start 61.98338335072809 51.5219035725218) (end 62.16506350946109 51.25) (stroke (width .05) (type default)) (layer "Edge.Cuts"))
 (gr_line (start 62.16506350946109 51.25) (end 62.30969883127822 50.956708580912725) (stroke (width .05) (type default)) (layer "Edge.Cuts"))
 (gr_line (start 62.30969883127822 50.956708580912725) (end 62.41481456572267 50.6470476127563) (stroke (width .05) (type default))
  (layer "Edge.Cuts"))
 (gr_line (start 62.41481456572267 50.6470476127563) (end 62.478612153434526 50.32631548055013) (stroke (width .05) (type default))
  (layer "Edge.Cuts"))
 (gr_line (start 62.478612153434526 50.32631548055013) (end 62.5 50.0) (stroke (width .05) (type default)) (layer "Edge.Cuts"))
 (gr_line (start 62.5 50.0) (end 62.478612153434526 49.67368451944987) (stroke (width .05) (type default)) (layer "Edge.Cuts"))
 (gr_line (start 62.478612153434526 49.67368451944987) (end 62.41481456572267 49.3529523872437) (stroke (width .05) (type default))
  (layer "Edge.Cuts"))
 (gr_line (start 62.41481456572267 49.3529523872437) (end 62.30969883127822 49.043291419087275) (stroke (width .05) (type default))
  (layer "Edge.Cuts"))
 (gr_line (start 62.30969883127822 49.043291419087275) (end 62.1650635094611 48.75) (stroke (width .05) (type default)) (layer "Edge.Cuts"))
 (gr_line (start 62.1650635094611 48.75) (end 61.98338335072809 48.4780964274782) (stroke (width .05) (type default)) (layer "Edge.Cuts"))
 (gr_line (start 61.98338335072809 48.4780964274782) (end 61.76776695296637 48.23223304703363) (stroke (width .05) (type default))
  (layer "Edge.Cuts"))
 (gr_line (start 61.76776695296637 48.23223304703363) (end 61.5219035725218 48.01661664927191) (stroke (width .05) (type default))
  (layer "Edge.Cuts"))
 (gr_line (start 61.5219035725218 48.01661664927191) (end 61.3 47.86834542243487) (stroke (width .05) (type default)) (layer "Edge.Cuts"))
 (gr_line (start 61.3 47.86834542243487) (end 61.3 46.7) (stroke (width .05) (type default)) (layer "Edge.Cuts"))
 (gr_line (start 61.3 46.7) (end 61.28887831978595 46.53031595011393) (stroke (width .05) (type default)) (layer "Edge.Cuts"))
 (gr_line (start 61.28887831978595 46.53031595011393) (end 61.25570357417579 46.363535241366726) (stroke (width .05) (type default))
  (layer "Edge.Cuts"))
 (gr_line (start 61.25570357417579 46.363535241366726) (end 61.20104339226467 46.20251153792538) (stroke (width .05) (type default))
  (layer "Edge.Cuts"))
 (gr_line (start 61.20104339226467 46.20251153792538) (end 61.12583302491977 46.05) (stroke (width .05) (type default)) (layer "Edge.Cuts"))
 (gr_line (start 61.12583302491977 46.05) (end 61.03135934237861 45.908610142288666) (stroke (width .05) (type default)) (layer "Edge.Cuts"))
 (gr_line (start 61.03135934237861 45.908610142288666) (end 60.91923881554251 45.78076118445749) (stroke (width .05) (type default))
  (layer "Edge.Cuts"))
 (gr_line (start 60.91923881554251 45.78076118445749) (end 60.79138985771134 45.668640657621395) (stroke (width .05) (type default))
  (layer "Edge.Cuts"))
 (gr_line (start 60.79138985771134 45.668640657621395) (end 60.65 45.57416697508023) (stroke (width .05) (type default)) (layer "Edge.Cuts"))
 (gr_line (start 60.65 45.57416697508023) (end 60.497488462074614 45.49895660773533) (stroke (width .05) (type default)) (layer "Edge.Cuts"))
 (gr_line (start 60.497488462074614 45.49895660773533) (end 60.33646475863328 45.44429642582421) (stroke (width .05) (type default))
  (layer "Edge.Cuts"))
 (gr_line (start 60.33646475863328 45.44429642582421) (end 60.169684049886065 45.411121680214045) (stroke (width .05) (type default))
  (layer "Edge.Cuts"))
 (gr_line (start 60.169684049886065 45.411121680214045) (end 60.16757283322946 45.410983303763615) (stroke (width .05) (type default))
  (layer "Edge.Cuts"))
 (gr_line (start 60.16757283322946 45.410983303763615) (end 60.07687846171137 44.9756503204768) (stroke (width .05) (type default))
  (layer "Edge.Cuts"))
 (gr_line (start 60.07687846171137 44.9756503204768) (end 60.0363181856797 44.831157732859225) (stroke (width .05) (type default))
  (layer "Edge.Cuts"))
 (gr_line (start 60.0363181856797 44.831157732859225) (end 59.97646762268844 44.69353086782984) (stroke (width .05) (type default))
  (layer "Edge.Cuts")))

